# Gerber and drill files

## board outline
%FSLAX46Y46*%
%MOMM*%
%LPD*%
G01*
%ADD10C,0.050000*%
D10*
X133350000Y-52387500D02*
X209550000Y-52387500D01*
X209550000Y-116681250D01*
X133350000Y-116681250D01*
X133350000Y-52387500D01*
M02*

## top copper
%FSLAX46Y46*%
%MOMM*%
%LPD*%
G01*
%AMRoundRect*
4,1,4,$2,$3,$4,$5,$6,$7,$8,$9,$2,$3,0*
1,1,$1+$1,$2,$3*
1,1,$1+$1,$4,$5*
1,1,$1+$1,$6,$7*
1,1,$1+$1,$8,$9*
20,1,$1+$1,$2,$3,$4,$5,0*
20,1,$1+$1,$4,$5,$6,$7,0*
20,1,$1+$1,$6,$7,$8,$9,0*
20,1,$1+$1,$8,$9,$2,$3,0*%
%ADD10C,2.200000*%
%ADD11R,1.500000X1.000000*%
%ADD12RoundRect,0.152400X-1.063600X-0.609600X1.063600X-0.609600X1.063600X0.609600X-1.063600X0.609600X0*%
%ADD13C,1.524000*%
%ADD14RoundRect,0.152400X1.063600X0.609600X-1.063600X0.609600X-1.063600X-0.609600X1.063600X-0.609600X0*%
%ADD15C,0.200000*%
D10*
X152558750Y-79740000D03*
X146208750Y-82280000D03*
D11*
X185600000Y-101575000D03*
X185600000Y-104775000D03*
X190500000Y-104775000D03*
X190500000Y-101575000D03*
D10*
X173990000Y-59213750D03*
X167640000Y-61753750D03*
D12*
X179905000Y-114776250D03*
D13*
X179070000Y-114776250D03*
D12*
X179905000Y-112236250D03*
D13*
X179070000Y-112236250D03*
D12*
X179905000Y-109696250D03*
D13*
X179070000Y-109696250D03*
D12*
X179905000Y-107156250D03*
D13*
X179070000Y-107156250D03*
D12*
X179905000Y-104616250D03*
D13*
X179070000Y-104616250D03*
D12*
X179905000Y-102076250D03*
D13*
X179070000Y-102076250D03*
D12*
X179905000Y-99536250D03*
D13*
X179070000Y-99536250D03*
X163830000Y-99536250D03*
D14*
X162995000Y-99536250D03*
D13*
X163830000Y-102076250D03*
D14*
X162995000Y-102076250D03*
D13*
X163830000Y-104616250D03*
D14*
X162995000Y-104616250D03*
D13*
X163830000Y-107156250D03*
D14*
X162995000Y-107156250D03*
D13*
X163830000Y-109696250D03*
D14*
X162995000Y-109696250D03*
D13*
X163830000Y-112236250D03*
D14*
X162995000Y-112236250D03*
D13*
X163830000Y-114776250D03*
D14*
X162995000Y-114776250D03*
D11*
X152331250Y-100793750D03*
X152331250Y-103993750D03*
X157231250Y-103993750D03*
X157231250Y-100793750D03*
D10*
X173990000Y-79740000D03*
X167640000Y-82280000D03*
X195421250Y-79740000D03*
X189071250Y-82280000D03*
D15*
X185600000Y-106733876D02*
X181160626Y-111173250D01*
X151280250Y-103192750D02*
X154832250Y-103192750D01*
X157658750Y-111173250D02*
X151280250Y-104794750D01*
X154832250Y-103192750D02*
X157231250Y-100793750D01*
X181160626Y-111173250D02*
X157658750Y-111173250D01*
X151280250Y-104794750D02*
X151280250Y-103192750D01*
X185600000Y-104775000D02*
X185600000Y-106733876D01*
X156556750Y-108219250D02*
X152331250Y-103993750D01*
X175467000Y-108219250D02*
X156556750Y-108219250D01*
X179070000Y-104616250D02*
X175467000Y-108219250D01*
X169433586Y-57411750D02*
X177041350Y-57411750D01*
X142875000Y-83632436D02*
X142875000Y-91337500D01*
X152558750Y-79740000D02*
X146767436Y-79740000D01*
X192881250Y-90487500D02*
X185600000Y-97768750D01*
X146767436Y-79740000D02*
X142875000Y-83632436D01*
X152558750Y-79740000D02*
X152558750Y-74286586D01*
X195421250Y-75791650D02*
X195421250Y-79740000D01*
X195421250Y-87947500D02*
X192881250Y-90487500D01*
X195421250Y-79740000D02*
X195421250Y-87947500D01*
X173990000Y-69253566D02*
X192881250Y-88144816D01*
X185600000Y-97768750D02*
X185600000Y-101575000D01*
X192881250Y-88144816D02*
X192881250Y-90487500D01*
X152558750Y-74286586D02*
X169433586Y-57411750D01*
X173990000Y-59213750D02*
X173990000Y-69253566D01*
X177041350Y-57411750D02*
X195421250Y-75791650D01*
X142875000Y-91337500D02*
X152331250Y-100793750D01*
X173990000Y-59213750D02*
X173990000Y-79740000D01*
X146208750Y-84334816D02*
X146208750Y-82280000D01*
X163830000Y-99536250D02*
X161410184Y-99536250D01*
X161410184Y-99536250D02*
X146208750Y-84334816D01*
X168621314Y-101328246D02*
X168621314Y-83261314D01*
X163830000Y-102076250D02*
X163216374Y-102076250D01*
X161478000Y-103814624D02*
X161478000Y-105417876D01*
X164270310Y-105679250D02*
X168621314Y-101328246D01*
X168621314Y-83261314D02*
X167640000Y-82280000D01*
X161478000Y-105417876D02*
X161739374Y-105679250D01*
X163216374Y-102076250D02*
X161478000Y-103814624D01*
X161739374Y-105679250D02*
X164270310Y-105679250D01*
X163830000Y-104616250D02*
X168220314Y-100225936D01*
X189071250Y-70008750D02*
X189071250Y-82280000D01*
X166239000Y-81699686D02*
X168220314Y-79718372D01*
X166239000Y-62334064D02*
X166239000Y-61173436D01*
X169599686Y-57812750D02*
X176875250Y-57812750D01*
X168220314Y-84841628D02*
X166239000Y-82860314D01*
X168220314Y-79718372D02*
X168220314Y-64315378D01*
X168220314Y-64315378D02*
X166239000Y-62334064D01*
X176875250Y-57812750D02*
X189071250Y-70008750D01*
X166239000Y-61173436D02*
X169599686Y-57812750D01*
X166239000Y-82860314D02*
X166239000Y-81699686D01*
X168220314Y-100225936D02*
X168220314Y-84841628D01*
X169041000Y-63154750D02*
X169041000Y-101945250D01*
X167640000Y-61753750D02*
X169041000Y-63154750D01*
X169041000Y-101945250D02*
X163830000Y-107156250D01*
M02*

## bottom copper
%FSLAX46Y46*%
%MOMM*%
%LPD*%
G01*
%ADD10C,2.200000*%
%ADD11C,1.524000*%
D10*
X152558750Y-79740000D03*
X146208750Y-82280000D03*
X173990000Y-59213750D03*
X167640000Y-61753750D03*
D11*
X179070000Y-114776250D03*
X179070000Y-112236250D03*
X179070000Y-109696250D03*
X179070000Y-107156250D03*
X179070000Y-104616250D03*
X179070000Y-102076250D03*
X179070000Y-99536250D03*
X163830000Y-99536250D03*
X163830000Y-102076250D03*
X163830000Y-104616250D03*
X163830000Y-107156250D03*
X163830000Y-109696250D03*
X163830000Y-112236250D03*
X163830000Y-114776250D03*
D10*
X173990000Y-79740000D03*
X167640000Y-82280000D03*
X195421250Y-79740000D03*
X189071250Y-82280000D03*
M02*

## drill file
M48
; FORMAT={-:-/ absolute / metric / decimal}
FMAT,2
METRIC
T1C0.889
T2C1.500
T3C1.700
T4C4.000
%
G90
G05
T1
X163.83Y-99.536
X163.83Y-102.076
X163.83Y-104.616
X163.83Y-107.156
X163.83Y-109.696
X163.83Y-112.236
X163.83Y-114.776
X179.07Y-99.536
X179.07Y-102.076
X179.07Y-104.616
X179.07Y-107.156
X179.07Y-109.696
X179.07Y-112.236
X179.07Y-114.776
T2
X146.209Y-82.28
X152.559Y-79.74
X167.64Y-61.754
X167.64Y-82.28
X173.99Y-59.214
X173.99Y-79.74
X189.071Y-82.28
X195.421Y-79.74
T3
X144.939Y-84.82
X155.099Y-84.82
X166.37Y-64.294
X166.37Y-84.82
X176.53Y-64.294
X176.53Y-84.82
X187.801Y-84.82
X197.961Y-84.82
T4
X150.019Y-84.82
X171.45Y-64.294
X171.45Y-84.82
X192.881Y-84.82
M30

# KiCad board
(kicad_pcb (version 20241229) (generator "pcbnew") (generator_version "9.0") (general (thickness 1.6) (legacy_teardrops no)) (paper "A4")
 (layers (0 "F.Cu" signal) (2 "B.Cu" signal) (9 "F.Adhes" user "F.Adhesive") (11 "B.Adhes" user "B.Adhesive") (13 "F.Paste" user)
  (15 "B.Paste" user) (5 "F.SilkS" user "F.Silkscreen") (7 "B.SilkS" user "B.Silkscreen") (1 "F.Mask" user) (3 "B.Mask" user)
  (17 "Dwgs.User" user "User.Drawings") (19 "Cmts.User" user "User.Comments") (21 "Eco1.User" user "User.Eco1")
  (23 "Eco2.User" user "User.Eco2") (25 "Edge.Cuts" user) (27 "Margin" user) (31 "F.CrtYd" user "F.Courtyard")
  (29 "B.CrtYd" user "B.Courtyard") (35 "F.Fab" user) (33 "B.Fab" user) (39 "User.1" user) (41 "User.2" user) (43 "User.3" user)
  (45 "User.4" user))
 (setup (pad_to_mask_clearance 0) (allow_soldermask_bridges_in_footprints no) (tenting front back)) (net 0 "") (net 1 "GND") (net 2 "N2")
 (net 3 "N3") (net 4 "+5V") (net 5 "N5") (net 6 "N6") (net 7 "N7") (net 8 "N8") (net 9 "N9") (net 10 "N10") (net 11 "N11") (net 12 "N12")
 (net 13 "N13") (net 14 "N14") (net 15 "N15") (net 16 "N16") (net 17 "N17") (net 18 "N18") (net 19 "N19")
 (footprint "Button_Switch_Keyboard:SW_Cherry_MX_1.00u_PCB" (layer "F.Cu") (at 152.55875 79.74)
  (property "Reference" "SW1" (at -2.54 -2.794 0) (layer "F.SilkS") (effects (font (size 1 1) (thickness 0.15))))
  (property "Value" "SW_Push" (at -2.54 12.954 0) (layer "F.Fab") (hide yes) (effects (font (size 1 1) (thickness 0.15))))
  (pad "" np_thru_hole circle (at -7.62 5.08) (size 1.7 1.7) (drill 1.7) (layers "*.Cu" "*.Mask"))
  (pad "" np_thru_hole circle (at -2.54 5.08) (size 4 4) (drill 4) (layers "*.Cu" "*.Mask"))
  (pad "" np_thru_hole circle (at 2.54 5.08) (size 1.7 1.7) (drill 1.7) (layers "*.Cu" "*.Mask"))
  (pad "1" thru_hole circle (at 0 0) (size 2.2 2.2) (drill 1.5) (layers "*.Cu" "*.Mask") (remove_unused_layers no) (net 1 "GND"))
  (pad "2" thru_hole circle (at -6.35 2.54) (size 2.2 2.2) (drill 1.5) (layers "*.Cu" "*.Mask") (remove_unused_layers no) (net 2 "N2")))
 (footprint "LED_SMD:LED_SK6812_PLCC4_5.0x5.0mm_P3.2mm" (layer "F.Cu") (at 188.05 103.175)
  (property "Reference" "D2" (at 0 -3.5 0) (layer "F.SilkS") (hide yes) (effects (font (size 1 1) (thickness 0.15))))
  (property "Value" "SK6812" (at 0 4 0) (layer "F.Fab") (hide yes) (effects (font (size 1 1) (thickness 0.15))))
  (pad "1" smd rect (at -2.45 -1.6 180) (size 1.5 1) (layers "F.Cu" "F.Mask" "F.Paste") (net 1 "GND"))
  (pad "2" smd rect (at -2.45 1.6 180) (size 1.5 1) (layers "F.Cu" "F.Mask" "F.Paste") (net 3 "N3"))
  (pad "3" smd rect (at 2.45 1.6 180) (size 1.5 1) (layers "F.Cu" "F.Mask" "F.Paste") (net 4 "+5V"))
  (pad "4" smd rect (at 2.45 -1.6 180) (size 1.5 1) (layers "F.Cu" "F.Mask" "F.Paste") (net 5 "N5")))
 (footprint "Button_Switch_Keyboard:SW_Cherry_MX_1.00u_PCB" (layer "F.Cu") (at 173.99 59.21375)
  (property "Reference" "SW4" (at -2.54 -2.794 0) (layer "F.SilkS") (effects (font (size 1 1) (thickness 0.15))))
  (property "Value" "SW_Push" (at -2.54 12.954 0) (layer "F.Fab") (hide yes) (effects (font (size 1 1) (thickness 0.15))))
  (pad "" np_thru_hole circle (at -7.62 5.08) (size 1.7 1.7) (drill 1.7) (layers "*.Cu" "*.Mask"))
  (pad "" np_thru_hole circle (at -2.54 5.08) (size 4 4) (drill 4) (layers "*.Cu" "*.Mask"))
  (pad "" np_thru_hole circle (at 2.54 5.08) (size 1.7 1.7) (drill 1.7) (layers "*.Cu" "*.Mask"))
  (pad "1" thru_hole circle (at 0 0) (size 2.2 2.2) (drill 1.5) (layers "*.Cu" "*.Mask") (remove_unused_layers no) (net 1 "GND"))
  (pad "2" thru_hole circle (at -6.35 2.54) (size 2.2 2.2) (drill 1.5) (layers "*.Cu" "*.Mask") (remove_unused_layers no) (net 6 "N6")))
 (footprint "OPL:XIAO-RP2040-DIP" (layer "F.Cu") (at 171.45 107.15625 180)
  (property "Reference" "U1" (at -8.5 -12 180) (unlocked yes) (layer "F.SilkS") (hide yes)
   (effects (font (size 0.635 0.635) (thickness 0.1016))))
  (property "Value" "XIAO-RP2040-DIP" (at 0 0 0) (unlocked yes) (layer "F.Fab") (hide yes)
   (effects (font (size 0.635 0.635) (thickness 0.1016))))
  (pad "1" smd roundrect (at -8.455 -7.62) (size 2.432 1.524) (layers "F.Cu" "F.Mask") (roundrect_rratio 0.1) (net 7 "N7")
   (thermal_bridge_angle 45))
  (pad "1" thru_hole circle (at -7.62 -7.62) (size 1.524 1.524) (drill 0.889) (layers "*.Cu" "*.Mask") (remove_unused_layers no)
   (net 7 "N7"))
  (pad "2" smd roundrect (at -8.455 -5.08) (size 2.432 1.524) (layers "F.Cu" "F.Mask") (roundrect_rratio 0.1) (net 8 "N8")
   (thermal_bridge_angle 45))
  (pad "2" thru_hole circle (at -7.62 -5.08) (size 1.524 1.524) (drill 0.889) (layers "*.Cu" "*.Mask") (remove_unused_layers no)
   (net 8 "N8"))
  (pad "3" smd roundrect (at -8.455 -2.54) (size 2.432 1.524) (layers "F.Cu" "F.Mask") (roundrect_rratio 0.1) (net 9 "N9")
   (thermal_bridge_angle 45))
  (pad "3" thru_hole circle (at -7.62 -2.54) (size 1.524 1.524) (drill 0.889) (layers "*.Cu" "*.Mask") (remove_unused_layers no)
   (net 9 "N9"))
  (pad "4" smd roundrect (at -8.455 0) (size 2.432 1.524) (layers "F.Cu" "F.Mask") (roundrect_rratio 0.1) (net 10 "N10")
   (thermal_bridge_angle 45))
  (pad "4" thru_hole circle (at -7.62 0) (size 1.524 1.524) (drill 0.889) (layers "*.Cu" "*.Mask") (remove_unused_layers no) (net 10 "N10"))
  (pad "5" smd roundrect (at -8.455 2.54) (size 2.432 1.524) (layers "F.Cu" "F.Mask") (roundrect_rratio 0.1) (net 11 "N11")
   (thermal_bridge_angle 45))
  (pad "5" thru_hole circle (at -7.62 2.54) (size 1.524 1.524) (drill 0.889) (layers "*.Cu" "*.Mask") (remove_unused_layers no)
   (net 11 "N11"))
  (pad "6" smd roundrect (at -8.455 5.08) (size 2.432 1.524) (layers "F.Cu" "F.Mask") (roundrect_rratio 0.1) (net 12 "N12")
   (thermal_bridge_angle 45))
  (pad "6" thru_hole circle (at -7.62 5.08) (size 1.524 1.524) (drill 0.889) (layers "*.Cu" "*.Mask") (remove_unused_layers no)
   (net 12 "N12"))
  (pad "7" smd roundrect (at -8.455 7.62) (size 2.432 1.524) (layers "F.Cu" "F.Mask") (roundrect_rratio 0.1) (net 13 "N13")
   (thermal_bridge_angle 45))
  (pad "7" thru_hole circle (at -7.62 7.62) (size 1.524 1.524) (drill 0.889) (layers "*.Cu" "*.Mask") (remove_unused_layers no)
   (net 13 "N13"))
  (pad "8" thru_hole circle (at 7.62 7.62 180) (size 1.524 1.524) (drill 0.889) (layers "*.Cu" "*.Mask") (remove_unused_layers no)
   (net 2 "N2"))
  (pad "8" smd roundrect (at 8.455 7.62 180) (size 2.432 1.524) (layers "F.Cu" "F.Mask") (roundrect_rratio 0.1) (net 2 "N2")
   (thermal_bridge_angle 45))
  (pad "9" thru_hole circle (at 7.62 5.08 180) (size 1.524 1.524) (drill 0.889) (layers "*.Cu" "*.Mask") (remove_unused_layers no)
   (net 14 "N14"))
  (pad "9" smd roundrect (at 8.455 5.08 180) (size 2.432 1.524) (layers "F.Cu" "F.Mask") (roundrect_rratio 0.1) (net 14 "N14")
   (thermal_bridge_angle 45))
  (pad "10" thru_hole circle (at 7.62 2.54 180) (size 1.524 1.524) (drill 0.889) (layers "*.Cu" "*.Mask") (remove_unused_layers no)
   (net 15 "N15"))
  (pad "10" smd roundrect (at 8.455 2.54 180) (size 2.432 1.524) (layers "F.Cu" "F.Mask") (roundrect_rratio 0.1) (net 15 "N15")
   (thermal_bridge_angle 45))
  (pad "11" thru_hole circle (at 7.62 0 180) (size 1.524 1.524) (drill 0.889) (layers "*.Cu" "*.Mask") (remove_unused_layers no)
   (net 6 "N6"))
  (pad "11" smd roundrect (at 8.455 0 180) (size 2.432 1.524) (layers "F.Cu" "F.Mask") (roundrect_rratio 0.1) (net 6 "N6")
   (thermal_bridge_angle 45))
  (pad "12" thru_hole circle (at 7.62 -2.54 180) (size 1.524 1.524) (drill 0.889) (layers "*.Cu" "*.Mask") (remove_unused_layers no)
   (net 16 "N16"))
  (pad "12" smd roundrect (at 8.455 -2.54 180) (size 2.432 1.524) (layers "F.Cu" "F.Mask") (roundrect_rratio 0.1) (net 16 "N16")
   (thermal_bridge_angle 45))
  (pad "13" thru_hole circle (at 7.62 -5.08 180) (size 1.524 1.524) (drill 0.889) (layers "*.Cu" "*.Mask") (remove_unused_layers no)
   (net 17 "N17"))
  (pad "13" smd roundrect (at 8.455 -5.08 180) (size 2.432 1.524) (layers "F.Cu" "F.Mask") (roundrect_rratio 0.1) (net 17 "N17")
   (thermal_bridge_angle 45))
  (pad "14" thru_hole circle (at 7.62 -7.62 180) (size 1.524 1.524) (drill 0.889) (layers "*.Cu" "*.Mask") (remove_unused_layers no)
   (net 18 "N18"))
  (pad "14" smd roundrect (at 8.455 -7.62 180) (size 2.432 1.524) (layers "F.Cu" "F.Mask") (roundrect_rratio 0.1) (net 18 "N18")
   (thermal_bridge_angle 45)))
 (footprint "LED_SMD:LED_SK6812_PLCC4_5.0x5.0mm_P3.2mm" (layer "F.Cu") (at 154.78125 102.39375)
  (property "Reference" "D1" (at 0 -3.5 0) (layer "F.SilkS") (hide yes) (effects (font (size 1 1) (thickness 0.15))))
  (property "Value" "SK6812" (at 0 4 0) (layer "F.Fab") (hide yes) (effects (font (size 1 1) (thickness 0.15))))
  (pad "1" smd rect (at -2.45 -1.6 180) (size 1.5 1) (layers "F.Cu" "F.Mask" "F.Paste") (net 1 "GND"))
  (pad "2" smd rect (at -2.45 1.6 180) (size 1.5 1) (layers "F.Cu" "F.Mask" "F.Paste") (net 11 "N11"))
  (pad "3" smd rect (at 2.45 1.6 180) (size 1.5 1) (layers "F.Cu" "F.Mask" "F.Paste") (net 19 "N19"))
  (pad "4" smd rect (at 2.45 -1.6 180) (size 1.5 1) (layers "F.Cu" "F.Mask" "F.Paste") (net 3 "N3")))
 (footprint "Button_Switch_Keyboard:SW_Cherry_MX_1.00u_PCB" (layer "F.Cu") (at 173.99 79.74)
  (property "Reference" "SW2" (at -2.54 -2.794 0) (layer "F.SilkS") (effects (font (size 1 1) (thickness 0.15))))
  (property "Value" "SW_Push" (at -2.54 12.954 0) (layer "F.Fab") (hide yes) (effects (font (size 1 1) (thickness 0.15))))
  (pad "" np_thru_hole circle (at -7.62 5.08) (size 1.7 1.7) (drill 1.7) (layers "*.Cu" "*.Mask"))
  (pad "" np_thru_hole circle (at -2.54 5.08) (size 4 4) (drill 4) (layers "*.Cu" "*.Mask"))
  (pad "" np_thru_hole circle (at 2.54 5.08) (size 1.7 1.7) (drill 1.7) (layers "*.Cu" "*.Mask"))
  (pad "1" thru_hole circle (at 0 0) (size 2.2 2.2) (drill 1.5) (layers "*.Cu" "*.Mask") (remove_unused_layers no) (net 1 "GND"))
  (pad "2" thru_hole circle (at -6.35 2.54) (size 2.2 2.2) (drill 1.5) (layers "*.Cu" "*.Mask") (remove_unused_layers no) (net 14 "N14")))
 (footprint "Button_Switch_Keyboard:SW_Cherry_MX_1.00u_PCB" (layer "F.Cu") (at 195.42125 79.74)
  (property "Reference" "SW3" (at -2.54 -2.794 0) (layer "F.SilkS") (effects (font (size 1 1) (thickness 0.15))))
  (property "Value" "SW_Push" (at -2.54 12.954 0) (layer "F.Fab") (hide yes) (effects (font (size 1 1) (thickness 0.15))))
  (pad "" np_thru_hole circle (at -7.62 5.08) (size 1.7 1.7) (drill 1.7) (layers "*.Cu" "*.Mask"))
  (pad "" np_thru_hole circle (at -2.54 5.08) (size 4 4) (drill 4) (layers "*.Cu" "*.Mask"))
  (pad "" np_thru_hole circle (at 2.54 5.08) (size 1.7 1.7) (drill 1.7) (layers "*.Cu" "*.Mask"))
  (pad "1" thru_hole circle (at 0 0) (size 2.2 2.2) (drill 1.5) (layers "*.Cu" "*.Mask") (remove_unused_layers no) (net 1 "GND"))
  (pad "2" thru_hole circle (at -6.35 2.54) (size 2.2 2.2) (drill 1.5) (layers "*.Cu" "*.Mask") (remove_unused_layers no) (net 15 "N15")))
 (gr_rect (start 133.35 52.3875) (end 209.55 116.68125) (stroke (width 0.05) (type default)) (fill no) (layer "Edge.Cuts"))
 (segment (start 185.6 106.733876) (end 181.160626 111.17325) (width 0.2) (layer "F.Cu") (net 3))
 (segment (start 151.28025 103.19275) (end 154.83225 103.19275) (width 0.2) (layer "F.Cu") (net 3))
 (segment (start 157.65875 111.17325) (end 151.28025 104.79475) (width 0.2) (layer "F.Cu") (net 3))
 (segment (start 154.83225 103.19275) (end 157.23125 100.79375) (width 0.2) (layer "F.Cu") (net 3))
 (segment (start 181.160626 111.17325) (end 157.65875 111.17325) (width 0.2) (layer "F.Cu") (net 3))
 (segment (start 151.28025 104.79475) (end 151.28025 103.19275) (width 0.2) (layer "F.Cu") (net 3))
 (segment (start 185.6 104.775) (end 185.6 106.733876) (width 0.2) (layer "F.Cu") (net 3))
 (segment (start 156.55675 108.21925) (end 152.33125 103.99375) (width 0.2) (layer "F.Cu") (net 11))
 (segment (start 175.467 108.21925) (end 156.55675 108.21925) (width 0.2) (layer "F.Cu") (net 11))
 (segment (start 179.07 104.61625) (end 175.467 108.21925) (width 0.2) (layer "F.Cu") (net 11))
 (segment (start 169.433586 57.41175) (end 177.04135 57.41175) (width 0.2) (layer "F.Cu") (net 1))
 (segment (start 142.875 83.632436) (end 142.875 91.3375) (width 0.2) (layer "F.Cu") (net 1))
 (segment (start 152.55875 79.74) (end 146.767436 79.74) (width 0.2) (layer "F.Cu") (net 1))
 (segment (start 192.88125 90.4875) (end 185.6 97.76875) (width 0.2) (layer "F.Cu") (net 1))
 (segment (start 146.767436 79.74) (end 142.875 83.632436) (width 0.2) (layer "F.Cu") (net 1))
 (segment (start 152.55875 79.74) (end 152.55875 74.286586) (width 0.2) (layer "F.Cu") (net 1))
 (segment (start 195.42125 75.79165) (end 195.42125 79.74) (width 0.2) (layer "F.Cu") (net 1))
 (segment (start 195.42125 87.9475) (end 192.88125 90.4875) (width 0.2) (layer "F.Cu") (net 1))
 (segment (start 195.42125 79.74) (end 195.42125 87.9475) (width 0.2) (layer "F.Cu") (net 1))
 (segment (start 173.99 69.253566) (end 192.88125 88.144816) (width 0.2) (layer "F.Cu") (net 1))
 (segment (start 185.6 97.76875) (end 185.6 101.575) (width 0.2) (layer "F.Cu") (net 1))
 (segment (start 192.88125 88.144816) (end 192.88125 90.4875) (width 0.2) (layer "F.Cu") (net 1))
 (segment (start 152.55875 74.286586) (end 169.433586 57.41175) (width 0.2) (layer "F.Cu") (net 1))
 (segment (start 173.99 59.21375) (end 173.99 69.253566) (width 0.2) (layer "F.Cu") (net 1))
 (segment (start 177.04135 57.41175) (end 195.42125 75.79165) (width 0.2) (layer "F.Cu") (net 1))
 (segment (start 142.875 91.3375) (end 152.33125 100.79375) (width 0.2) (layer "F.Cu") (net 1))
 (segment (start 173.99 59.21375) (end 173.99 79.74) (width 0.2) (layer "F.Cu") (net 1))
 (segment (start 146.20875 84.334816) (end 146.20875 82.28) (width 0.2) (layer "F.Cu") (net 2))
 (segment (start 163.83 99.53625) (end 161.410184 99.53625) (width 0.2) (layer "F.Cu") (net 2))
 (segment (start 161.410184 99.53625) (end 146.20875 84.334816) (width 0.2) (layer "F.Cu") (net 2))
 (segment (start 168.621314 101.328246) (end 168.621314 83.261314) (width 0.2) (layer "F.Cu") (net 14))
 (segment (start 163.83 102.07625) (end 163.216374 102.07625) (width 0.2) (layer "F.Cu") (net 14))
 (segment (start 161.478 103.814624) (end 161.478 105.417876) (width 0.2) (layer "F.Cu") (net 14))
 (segment (start 164.27031 105.67925) (end 168.621314 101.328246) (width 0.2) (layer "F.Cu") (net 14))
 (segment (start 168.621314 83.261314) (end 167.64 82.28) (width 0.2) (layer "F.Cu") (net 14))
 (segment (start 161.478 105.417876) (end 161.739374 105.67925) (width 0.2) (layer "F.Cu") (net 14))
 (segment (start 163.216374 102.07625) (end 161.478 103.814624) (width 0.2) (layer "F.Cu") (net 14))
 (segment (start 161.739374 105.67925) (end 164.27031 105.67925) (width 0.2) (layer "F.Cu") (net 14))
 (segment (start 163.83 104.61625) (end 168.220314 100.225936) (width 0.2) (layer "F.Cu") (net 15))
 (segment (start 189.07125 70.00875) (end 189.07125 82.28) (width 0.2) (layer "F.Cu") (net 15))
 (segment (start 166.239 81.699686) (end 168.220314 79.718372) (width 0.2) (layer "F.Cu") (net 15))
 (segment (start 166.239 62.334064) (end 166.239 61.173436) (width 0.2) (layer "F.Cu") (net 15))
 (segment (start 169.599686 57.81275) (end 176.87525 57.81275) (width 0.2) (layer "F.Cu") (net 15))
 (segment (start 168.220314 84.841628) (end 166.239 82.860314) (width 0.2) (layer "F.Cu") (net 15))
 (segment (start 168.220314 79.718372) (end 168.220314 64.315378) (width 0.2) (layer "F.Cu") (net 15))
 (segment (start 168.220314 64.315378) (end 166.239 62.334064) (width 0.2) (layer "F.Cu") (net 15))
 (segment (start 176.87525 57.81275) (end 189.07125 70.00875) (width 0.2) (layer "F.Cu") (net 15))
 (segment (start 166.239 61.173436) (end 169.599686 57.81275) (width 0.2) (layer "F.Cu") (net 15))
 (segment (start 166.239 82.860314) (end 166.239 81.699686) (width 0.2) (layer "F.Cu") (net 15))
 (segment (start 168.220314 100.225936) (end 168.220314 84.841628) (width 0.2) (layer "F.Cu") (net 15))
 (segment (start 169.041 63.15475) (end 169.041 101.94525) (width 0.2) (layer "F.Cu") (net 6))
 (segment (start 167.64 61.75375) (end 169.041 63.15475) (width 0.2) (layer "F.Cu") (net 6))
 (segment (start 169.041 101.94525) (end 163.83 107.15625) (width 0.2) (layer "F.Cu") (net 6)))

